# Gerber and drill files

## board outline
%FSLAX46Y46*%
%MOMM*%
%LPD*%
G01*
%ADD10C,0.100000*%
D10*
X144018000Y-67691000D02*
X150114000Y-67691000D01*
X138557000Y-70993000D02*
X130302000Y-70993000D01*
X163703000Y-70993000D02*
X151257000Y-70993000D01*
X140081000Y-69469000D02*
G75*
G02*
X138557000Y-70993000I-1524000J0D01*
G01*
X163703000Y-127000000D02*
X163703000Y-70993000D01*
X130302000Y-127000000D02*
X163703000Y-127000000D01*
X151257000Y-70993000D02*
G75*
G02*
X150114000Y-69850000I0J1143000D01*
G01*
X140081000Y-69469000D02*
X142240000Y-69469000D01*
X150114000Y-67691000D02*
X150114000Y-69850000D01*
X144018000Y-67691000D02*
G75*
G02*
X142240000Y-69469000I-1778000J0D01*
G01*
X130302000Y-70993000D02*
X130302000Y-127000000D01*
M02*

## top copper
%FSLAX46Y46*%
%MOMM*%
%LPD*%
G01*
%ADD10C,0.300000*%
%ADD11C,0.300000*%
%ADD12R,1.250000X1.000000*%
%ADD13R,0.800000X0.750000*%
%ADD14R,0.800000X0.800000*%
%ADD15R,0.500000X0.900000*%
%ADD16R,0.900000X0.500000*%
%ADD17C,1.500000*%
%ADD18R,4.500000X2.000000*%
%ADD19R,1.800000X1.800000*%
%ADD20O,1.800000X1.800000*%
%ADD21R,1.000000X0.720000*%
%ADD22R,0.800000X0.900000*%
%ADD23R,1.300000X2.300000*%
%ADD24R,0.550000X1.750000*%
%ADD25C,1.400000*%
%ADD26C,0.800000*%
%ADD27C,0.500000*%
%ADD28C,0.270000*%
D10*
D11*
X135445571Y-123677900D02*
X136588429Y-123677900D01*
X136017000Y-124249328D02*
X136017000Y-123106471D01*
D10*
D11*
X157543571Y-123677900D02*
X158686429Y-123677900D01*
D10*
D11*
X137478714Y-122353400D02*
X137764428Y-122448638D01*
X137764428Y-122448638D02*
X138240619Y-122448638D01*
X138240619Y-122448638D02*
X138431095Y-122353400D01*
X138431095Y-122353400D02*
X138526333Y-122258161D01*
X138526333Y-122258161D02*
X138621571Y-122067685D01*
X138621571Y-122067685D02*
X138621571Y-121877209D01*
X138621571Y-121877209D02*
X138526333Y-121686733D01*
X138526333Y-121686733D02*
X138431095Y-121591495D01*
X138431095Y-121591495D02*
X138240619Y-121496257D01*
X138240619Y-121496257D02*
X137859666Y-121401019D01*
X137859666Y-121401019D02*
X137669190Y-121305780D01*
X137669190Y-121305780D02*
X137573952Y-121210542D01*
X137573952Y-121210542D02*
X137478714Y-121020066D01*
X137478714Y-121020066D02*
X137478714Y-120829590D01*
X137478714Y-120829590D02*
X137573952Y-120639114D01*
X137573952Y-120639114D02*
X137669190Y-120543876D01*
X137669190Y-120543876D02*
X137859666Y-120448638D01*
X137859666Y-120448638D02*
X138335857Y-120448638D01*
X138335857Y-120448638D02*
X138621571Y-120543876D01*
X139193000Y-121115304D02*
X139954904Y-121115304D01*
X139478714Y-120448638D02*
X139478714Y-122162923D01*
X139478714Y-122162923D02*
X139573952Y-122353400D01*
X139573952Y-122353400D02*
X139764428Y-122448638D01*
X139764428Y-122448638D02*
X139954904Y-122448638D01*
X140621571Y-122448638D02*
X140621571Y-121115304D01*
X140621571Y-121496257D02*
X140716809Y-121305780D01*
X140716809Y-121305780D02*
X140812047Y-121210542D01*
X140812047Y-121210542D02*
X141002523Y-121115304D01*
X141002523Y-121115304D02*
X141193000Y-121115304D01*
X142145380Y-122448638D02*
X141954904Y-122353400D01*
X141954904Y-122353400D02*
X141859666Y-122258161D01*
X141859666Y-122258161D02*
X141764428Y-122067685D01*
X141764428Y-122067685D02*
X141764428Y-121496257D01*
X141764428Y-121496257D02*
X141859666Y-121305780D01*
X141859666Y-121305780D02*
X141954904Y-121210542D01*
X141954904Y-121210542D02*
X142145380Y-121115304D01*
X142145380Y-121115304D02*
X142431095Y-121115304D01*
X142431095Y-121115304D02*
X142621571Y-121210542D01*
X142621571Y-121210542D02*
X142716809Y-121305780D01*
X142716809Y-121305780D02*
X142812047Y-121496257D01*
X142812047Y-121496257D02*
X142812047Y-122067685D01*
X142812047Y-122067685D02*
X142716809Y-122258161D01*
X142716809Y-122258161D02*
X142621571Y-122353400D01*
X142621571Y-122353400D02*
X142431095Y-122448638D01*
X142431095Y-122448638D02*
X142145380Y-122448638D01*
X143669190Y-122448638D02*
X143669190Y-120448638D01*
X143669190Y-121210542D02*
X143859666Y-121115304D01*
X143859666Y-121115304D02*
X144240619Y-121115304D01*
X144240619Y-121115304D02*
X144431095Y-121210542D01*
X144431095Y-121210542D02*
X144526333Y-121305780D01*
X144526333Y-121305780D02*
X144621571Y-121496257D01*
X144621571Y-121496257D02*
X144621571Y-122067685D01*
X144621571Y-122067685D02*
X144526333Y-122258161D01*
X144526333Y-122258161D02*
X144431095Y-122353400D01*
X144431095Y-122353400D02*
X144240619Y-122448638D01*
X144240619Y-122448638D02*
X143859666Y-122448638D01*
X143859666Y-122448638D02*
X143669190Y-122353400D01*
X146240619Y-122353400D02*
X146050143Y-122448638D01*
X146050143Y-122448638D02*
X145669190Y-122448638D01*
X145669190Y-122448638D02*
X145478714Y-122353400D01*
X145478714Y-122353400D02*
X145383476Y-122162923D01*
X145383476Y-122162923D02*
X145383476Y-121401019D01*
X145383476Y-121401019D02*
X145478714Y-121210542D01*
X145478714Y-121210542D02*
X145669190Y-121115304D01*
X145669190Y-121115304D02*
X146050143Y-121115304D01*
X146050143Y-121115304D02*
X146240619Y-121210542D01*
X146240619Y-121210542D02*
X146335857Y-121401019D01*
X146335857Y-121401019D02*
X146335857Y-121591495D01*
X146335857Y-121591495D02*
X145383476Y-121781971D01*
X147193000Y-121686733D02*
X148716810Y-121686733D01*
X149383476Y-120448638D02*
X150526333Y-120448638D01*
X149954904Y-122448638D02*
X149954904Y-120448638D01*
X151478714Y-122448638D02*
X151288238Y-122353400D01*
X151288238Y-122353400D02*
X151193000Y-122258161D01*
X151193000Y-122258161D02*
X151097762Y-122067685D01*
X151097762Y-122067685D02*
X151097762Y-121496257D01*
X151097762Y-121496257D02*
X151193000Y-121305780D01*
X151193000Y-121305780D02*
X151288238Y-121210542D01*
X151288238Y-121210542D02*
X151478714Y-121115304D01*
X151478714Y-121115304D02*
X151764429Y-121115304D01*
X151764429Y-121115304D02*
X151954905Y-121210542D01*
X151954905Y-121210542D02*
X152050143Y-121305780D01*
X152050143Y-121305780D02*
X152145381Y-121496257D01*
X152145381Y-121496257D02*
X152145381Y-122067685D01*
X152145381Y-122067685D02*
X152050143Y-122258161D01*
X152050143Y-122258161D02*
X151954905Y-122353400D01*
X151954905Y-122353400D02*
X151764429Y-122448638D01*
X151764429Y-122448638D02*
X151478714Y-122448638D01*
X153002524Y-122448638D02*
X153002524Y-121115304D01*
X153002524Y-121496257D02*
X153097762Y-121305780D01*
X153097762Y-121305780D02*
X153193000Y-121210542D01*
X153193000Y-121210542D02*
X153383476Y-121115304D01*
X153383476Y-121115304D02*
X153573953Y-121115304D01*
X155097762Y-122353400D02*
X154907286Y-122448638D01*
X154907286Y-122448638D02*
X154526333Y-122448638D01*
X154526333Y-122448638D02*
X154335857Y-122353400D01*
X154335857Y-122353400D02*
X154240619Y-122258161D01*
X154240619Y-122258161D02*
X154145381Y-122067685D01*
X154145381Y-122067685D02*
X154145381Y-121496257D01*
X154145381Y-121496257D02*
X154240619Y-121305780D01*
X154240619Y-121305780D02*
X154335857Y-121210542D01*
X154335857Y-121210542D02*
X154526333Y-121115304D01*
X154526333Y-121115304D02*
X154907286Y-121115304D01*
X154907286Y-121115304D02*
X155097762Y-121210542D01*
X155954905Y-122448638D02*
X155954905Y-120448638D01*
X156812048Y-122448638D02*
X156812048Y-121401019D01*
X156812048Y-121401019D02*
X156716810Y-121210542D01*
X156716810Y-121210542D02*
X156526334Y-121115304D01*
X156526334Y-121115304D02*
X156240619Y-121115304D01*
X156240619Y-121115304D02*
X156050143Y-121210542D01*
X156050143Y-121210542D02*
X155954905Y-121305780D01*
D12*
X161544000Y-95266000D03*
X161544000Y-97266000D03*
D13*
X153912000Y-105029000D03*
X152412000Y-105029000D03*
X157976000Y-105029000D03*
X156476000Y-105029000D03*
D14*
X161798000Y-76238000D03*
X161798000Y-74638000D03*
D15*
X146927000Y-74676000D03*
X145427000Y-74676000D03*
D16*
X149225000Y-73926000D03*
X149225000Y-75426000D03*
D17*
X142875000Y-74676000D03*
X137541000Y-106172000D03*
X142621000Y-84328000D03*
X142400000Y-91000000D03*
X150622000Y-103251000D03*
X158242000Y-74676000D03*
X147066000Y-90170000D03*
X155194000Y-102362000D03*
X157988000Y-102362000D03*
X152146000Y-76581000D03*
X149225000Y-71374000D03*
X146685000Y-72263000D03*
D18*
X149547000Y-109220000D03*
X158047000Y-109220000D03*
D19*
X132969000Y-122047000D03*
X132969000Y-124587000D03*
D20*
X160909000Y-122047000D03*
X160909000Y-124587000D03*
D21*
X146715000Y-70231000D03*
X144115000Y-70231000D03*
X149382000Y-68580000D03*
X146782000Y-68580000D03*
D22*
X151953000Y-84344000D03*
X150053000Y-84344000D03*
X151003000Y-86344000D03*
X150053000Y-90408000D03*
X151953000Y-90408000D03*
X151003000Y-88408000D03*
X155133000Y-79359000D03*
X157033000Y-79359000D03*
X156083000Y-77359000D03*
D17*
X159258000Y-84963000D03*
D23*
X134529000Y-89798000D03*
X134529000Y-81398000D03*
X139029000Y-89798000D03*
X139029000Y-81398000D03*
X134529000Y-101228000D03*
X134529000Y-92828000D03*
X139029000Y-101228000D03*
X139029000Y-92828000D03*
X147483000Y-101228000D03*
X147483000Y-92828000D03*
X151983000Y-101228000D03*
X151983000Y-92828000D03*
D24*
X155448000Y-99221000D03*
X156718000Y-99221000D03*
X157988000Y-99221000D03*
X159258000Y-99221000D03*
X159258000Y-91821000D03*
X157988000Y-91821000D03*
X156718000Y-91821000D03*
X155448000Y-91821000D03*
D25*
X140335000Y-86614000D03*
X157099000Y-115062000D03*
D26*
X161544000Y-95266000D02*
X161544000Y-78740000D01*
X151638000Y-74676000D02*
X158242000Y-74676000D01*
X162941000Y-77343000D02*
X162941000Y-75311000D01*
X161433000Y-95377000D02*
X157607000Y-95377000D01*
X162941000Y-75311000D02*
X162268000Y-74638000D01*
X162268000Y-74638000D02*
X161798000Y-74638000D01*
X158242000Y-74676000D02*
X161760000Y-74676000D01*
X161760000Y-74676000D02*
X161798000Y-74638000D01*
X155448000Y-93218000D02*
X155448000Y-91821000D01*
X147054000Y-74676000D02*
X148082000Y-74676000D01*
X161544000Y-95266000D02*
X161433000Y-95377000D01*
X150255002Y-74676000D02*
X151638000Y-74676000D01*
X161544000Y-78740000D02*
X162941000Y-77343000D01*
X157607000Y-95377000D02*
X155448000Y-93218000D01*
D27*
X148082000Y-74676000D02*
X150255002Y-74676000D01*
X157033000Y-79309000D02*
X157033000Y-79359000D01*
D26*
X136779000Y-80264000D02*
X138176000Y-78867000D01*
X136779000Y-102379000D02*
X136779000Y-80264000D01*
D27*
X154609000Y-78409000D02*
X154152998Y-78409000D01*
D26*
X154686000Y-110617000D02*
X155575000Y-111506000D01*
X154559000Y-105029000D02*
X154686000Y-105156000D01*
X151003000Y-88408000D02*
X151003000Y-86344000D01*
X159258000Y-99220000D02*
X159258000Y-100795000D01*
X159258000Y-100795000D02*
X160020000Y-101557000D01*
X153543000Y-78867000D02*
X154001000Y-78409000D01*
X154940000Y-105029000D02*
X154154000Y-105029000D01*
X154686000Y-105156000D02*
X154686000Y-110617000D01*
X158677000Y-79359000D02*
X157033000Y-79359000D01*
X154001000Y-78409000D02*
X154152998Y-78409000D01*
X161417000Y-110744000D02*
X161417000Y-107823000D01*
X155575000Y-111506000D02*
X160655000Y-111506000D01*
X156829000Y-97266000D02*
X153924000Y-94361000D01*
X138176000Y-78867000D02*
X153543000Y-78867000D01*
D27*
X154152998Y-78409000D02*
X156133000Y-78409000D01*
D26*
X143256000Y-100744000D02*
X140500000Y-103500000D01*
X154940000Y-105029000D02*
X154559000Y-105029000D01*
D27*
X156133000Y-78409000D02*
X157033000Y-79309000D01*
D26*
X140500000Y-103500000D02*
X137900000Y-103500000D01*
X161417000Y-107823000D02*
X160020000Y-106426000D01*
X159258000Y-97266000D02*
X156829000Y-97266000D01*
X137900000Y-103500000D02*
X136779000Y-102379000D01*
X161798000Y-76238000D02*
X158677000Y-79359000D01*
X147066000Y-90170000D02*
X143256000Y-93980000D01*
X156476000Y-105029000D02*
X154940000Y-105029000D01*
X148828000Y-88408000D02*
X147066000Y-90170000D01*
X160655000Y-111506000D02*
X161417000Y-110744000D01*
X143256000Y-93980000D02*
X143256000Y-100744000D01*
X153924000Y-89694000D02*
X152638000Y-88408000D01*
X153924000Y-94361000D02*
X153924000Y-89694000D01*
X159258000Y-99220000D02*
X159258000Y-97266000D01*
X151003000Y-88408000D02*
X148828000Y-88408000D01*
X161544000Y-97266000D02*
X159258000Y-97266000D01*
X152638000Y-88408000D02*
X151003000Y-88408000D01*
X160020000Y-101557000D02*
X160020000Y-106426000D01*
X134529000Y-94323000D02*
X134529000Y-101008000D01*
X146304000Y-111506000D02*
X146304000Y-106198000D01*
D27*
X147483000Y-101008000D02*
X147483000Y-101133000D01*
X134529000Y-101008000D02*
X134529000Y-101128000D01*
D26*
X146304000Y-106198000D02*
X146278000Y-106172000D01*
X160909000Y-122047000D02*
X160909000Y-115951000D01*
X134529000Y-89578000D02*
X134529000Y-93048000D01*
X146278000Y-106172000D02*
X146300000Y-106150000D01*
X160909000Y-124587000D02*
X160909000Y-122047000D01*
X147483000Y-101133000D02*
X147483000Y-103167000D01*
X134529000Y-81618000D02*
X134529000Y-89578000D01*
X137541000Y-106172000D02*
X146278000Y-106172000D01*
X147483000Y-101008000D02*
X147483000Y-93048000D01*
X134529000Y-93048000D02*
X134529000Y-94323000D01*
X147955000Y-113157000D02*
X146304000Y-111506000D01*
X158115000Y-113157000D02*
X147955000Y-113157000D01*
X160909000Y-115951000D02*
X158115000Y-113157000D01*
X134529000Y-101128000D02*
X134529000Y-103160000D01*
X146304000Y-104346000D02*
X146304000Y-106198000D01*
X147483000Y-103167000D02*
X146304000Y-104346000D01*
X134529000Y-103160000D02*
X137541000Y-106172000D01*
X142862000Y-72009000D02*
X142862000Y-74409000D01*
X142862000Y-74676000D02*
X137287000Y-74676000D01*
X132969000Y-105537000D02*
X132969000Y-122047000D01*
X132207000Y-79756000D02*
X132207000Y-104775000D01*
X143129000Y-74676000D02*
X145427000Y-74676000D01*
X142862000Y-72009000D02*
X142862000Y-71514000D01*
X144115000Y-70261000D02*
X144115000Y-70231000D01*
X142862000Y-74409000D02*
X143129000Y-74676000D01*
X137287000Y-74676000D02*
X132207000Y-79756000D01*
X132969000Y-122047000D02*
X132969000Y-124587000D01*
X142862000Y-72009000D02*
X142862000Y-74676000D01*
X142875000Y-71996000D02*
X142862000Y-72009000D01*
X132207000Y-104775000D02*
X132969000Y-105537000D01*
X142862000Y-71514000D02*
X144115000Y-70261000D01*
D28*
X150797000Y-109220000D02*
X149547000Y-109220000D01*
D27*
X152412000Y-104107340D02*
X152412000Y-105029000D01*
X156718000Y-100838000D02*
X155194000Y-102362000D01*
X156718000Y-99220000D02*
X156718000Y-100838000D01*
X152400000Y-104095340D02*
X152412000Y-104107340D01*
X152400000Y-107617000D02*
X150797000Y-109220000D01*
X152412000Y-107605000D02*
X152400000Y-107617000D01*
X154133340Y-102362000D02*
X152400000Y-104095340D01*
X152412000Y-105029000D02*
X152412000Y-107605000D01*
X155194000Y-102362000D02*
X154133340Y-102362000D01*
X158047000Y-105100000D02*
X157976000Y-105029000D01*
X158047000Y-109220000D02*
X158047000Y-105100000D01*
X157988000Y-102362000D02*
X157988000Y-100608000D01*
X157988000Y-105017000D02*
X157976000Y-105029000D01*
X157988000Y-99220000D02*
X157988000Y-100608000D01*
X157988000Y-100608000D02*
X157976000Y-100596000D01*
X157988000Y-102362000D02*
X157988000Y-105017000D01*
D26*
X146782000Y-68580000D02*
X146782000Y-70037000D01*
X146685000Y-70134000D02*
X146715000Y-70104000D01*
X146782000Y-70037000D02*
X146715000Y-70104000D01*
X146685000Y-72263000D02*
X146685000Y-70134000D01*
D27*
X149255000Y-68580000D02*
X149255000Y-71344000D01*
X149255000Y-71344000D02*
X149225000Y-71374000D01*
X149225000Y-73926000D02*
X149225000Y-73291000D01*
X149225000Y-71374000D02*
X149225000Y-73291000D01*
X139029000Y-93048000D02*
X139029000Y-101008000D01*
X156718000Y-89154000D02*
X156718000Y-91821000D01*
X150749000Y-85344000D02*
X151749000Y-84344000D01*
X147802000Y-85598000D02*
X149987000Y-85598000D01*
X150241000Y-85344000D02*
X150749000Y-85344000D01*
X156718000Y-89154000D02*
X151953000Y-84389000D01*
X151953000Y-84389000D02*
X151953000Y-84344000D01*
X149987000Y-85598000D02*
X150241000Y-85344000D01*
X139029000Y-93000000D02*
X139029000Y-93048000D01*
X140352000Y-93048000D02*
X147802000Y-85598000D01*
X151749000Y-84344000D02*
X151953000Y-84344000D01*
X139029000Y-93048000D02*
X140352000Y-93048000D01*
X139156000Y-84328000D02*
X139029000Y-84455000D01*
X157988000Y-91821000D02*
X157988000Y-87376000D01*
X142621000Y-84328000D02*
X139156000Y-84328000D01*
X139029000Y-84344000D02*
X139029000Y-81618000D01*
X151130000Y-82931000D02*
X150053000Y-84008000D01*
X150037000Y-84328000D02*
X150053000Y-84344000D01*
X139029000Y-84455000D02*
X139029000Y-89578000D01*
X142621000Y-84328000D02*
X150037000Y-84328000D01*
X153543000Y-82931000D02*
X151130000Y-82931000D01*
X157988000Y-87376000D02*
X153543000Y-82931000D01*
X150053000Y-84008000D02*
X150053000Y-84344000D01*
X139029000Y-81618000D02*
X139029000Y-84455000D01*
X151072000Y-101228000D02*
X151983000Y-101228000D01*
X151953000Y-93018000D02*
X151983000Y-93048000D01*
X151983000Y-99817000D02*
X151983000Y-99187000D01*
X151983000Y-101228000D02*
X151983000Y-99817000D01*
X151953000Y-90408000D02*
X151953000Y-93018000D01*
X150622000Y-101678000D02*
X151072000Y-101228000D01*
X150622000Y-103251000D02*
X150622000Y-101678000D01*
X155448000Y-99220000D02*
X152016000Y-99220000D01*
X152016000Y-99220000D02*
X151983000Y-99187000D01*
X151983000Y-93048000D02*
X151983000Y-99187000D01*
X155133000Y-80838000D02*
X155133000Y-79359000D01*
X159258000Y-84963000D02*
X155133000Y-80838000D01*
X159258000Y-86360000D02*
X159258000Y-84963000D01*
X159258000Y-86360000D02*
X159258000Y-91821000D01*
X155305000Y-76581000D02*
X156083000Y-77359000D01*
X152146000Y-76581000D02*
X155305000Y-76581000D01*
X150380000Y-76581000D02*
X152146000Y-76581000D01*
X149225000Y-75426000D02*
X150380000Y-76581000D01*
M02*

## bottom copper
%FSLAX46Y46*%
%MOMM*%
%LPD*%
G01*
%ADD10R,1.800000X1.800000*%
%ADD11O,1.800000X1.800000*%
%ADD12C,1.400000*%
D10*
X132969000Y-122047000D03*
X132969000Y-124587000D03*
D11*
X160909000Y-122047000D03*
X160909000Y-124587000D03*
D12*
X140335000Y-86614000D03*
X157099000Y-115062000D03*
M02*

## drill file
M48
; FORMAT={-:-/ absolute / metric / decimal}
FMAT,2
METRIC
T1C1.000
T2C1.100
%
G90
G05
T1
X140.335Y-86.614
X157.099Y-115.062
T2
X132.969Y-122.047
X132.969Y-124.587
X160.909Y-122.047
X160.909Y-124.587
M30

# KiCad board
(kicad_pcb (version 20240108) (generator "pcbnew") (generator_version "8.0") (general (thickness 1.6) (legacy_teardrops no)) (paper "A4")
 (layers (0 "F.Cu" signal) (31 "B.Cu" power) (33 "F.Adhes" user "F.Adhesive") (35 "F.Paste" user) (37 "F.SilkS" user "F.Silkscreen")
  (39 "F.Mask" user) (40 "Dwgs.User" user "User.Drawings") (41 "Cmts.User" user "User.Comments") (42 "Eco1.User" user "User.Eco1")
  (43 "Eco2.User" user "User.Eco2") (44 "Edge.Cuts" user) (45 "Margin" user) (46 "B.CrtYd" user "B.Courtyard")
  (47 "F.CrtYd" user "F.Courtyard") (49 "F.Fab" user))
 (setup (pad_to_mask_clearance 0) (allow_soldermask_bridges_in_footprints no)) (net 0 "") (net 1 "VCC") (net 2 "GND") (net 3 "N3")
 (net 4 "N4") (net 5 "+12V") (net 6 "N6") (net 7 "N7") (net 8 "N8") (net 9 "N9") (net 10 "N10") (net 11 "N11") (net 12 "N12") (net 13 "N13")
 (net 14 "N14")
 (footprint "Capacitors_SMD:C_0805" (layer "F.Cu") (at 161.544 96.266 -90)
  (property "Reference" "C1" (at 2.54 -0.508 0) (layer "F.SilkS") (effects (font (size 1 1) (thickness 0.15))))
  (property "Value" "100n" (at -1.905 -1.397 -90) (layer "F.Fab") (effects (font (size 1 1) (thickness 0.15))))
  (pad "1" smd rect (at -1 0 270) (size 1 1.25) (layers "F.Cu" "F.Paste" "F.Mask") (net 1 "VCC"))
  (pad "2" smd rect (at 1 0 270) (size 1 1.25) (layers "F.Cu" "F.Paste" "F.Mask") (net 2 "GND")))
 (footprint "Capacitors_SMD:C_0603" (layer "F.Cu") (at 153.162 105.029 180)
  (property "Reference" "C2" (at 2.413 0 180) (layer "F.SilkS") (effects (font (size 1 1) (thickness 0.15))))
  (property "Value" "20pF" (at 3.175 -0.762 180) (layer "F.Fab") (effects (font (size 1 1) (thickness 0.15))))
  (pad "1" smd rect (at -0.75 0 180) (size 0.8 0.75) (layers "F.Cu" "F.Paste" "F.Mask") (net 2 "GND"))
  (pad "2" smd rect (at 0.75 0 180) (size 0.8 0.75) (layers "F.Cu" "F.Paste" "F.Mask") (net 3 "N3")))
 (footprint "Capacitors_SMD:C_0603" (layer "F.Cu") (at 157.226 105.029 180)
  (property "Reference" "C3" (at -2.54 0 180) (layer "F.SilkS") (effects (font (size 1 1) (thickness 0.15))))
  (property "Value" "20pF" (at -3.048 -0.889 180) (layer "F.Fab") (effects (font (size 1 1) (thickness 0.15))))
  (pad "1" smd rect (at -0.75 0 180) (size 0.8 0.75) (layers "F.Cu" "F.Paste" "F.Mask") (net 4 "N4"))
  (pad "2" smd rect (at 0.75 0 180) (size 0.8 0.75) (layers "F.Cu" "F.Paste" "F.Mask") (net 2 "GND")))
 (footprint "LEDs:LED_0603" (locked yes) (layer "F.Cu") (at 161.798 75.438 90)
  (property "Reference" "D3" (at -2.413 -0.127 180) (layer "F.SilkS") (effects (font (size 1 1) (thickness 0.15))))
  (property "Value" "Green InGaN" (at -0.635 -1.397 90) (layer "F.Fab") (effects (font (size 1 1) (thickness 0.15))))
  (pad "1" smd rect (at -0.8 0 270) (size 0.8 0.8) (layers "F.Cu" "F.Paste" "F.Mask") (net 2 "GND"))
  (pad "2" smd rect (at 0.8 0 270) (size 0.8 0.8) (layers "F.Cu" "F.Paste" "F.Mask") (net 1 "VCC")))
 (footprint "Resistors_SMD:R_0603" (layer "F.Cu") (at 146.177 74.676 180)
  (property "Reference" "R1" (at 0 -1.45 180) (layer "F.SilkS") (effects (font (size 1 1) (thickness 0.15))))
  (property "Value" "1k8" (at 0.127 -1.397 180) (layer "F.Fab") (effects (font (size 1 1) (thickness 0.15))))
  (pad "1" smd rect (at -0.75 0 180) (size 0.5 0.9) (layers "F.Cu" "F.Paste" "F.Mask") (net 1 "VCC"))
  (pad "2" smd rect (at 0.75 0 180) (size 0.5 0.9) (layers "F.Cu" "F.Paste" "F.Mask") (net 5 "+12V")))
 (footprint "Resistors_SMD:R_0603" (layer "F.Cu") (at 149.225 74.676 -90)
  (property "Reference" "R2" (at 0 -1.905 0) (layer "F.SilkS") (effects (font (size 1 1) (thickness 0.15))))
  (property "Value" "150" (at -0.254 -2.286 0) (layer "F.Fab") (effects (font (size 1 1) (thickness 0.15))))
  (pad "1" smd rect (at -0.75 0 270) (size 0.5 0.9) (layers "F.Cu" "F.Paste" "F.Mask") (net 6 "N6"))
  (pad "2" smd rect (at 0.75 0 270) (size 0.5 0.9) (layers "F.Cu" "F.Paste" "F.Mask") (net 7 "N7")))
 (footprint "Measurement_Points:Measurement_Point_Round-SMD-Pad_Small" (layer "F.Cu") (at 142.875 74.676)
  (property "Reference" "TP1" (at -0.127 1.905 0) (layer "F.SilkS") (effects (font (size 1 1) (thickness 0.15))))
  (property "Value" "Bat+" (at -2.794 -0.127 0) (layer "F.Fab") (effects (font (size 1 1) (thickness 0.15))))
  (pad "1" smd circle (at 0 0) (size 1.5 1.5) (layers "F.Cu" "F.Mask") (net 5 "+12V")))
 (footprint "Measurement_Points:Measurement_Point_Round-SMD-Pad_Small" (layer "F.Cu") (at 137.541 106.172)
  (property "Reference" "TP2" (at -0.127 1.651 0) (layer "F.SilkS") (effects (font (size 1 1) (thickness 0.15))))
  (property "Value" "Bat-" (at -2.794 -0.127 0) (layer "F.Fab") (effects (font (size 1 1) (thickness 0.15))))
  (pad "1" smd circle (at 0 0) (size 1.5 1.5) (layers "F.Cu" "F.Mask") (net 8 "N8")))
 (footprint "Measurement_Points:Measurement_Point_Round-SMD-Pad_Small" (layer "F.Cu") (at 142.621 84.328)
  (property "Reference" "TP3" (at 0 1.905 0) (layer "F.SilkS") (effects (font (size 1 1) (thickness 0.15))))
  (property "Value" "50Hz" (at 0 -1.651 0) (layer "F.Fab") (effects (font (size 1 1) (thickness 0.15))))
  (pad "1" smd circle (at 0 0) (size 1.5 1.5) (layers "F.Cu" "F.Mask") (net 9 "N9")))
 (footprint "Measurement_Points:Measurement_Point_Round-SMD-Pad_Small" (layer "F.Cu") (at 142.4 91)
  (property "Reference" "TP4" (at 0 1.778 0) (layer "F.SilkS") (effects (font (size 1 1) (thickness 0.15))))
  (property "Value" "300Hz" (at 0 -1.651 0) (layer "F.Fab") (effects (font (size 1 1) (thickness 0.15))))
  (pad "1" smd circle (at 0 0) (size 1.5 1.5) (layers "F.Cu" "F.Mask") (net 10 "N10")))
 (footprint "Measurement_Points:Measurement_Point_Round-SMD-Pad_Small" (layer "F.Cu") (at 150.622 103.251)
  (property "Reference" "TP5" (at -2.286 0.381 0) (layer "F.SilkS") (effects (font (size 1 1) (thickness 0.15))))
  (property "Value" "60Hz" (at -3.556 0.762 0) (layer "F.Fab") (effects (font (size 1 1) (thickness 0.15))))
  (pad "1" smd circle (at 0 0) (size 1.5 1.5) (layers "F.Cu" "F.Mask") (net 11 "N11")))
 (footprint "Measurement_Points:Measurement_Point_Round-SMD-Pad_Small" (layer "F.Cu") (at 158.242 74.676)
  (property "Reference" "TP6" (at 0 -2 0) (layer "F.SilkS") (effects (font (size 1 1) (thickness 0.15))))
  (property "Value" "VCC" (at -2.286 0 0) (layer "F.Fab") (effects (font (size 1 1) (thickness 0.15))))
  (pad "1" smd circle (at 0 0) (size 1.5 1.5) (layers "F.Cu" "F.Mask") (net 1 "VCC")))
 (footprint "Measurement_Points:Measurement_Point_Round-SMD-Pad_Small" (layer "F.Cu") (at 147.066 90.17)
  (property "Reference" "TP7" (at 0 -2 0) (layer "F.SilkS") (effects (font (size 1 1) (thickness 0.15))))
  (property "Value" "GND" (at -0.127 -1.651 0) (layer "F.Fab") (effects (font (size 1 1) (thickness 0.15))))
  (pad "1" smd circle (at 0 0) (size 1.5 1.5) (layers "F.Cu" "F.Mask") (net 2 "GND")))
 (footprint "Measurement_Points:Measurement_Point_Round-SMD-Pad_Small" (layer "F.Cu") (at 155.194 102.362)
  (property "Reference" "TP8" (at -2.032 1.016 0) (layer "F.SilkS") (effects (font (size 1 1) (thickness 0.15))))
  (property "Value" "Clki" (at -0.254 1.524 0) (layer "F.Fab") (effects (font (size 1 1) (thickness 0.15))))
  (pad "1" smd circle (at 0 0) (size 1.5 1.5) (layers "F.Cu" "F.Mask") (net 3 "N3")))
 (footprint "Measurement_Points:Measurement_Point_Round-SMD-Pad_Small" (layer "F.Cu") (at 157.988 102.362)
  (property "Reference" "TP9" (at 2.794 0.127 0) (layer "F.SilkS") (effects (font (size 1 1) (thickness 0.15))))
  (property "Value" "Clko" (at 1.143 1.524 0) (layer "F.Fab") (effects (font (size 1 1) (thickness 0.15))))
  (pad "1" smd circle (at 0 0) (size 1.5 1.5) (layers "F.Cu" "F.Mask") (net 4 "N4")))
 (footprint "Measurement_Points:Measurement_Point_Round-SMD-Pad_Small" (layer "F.Cu") (at 152.146 76.581)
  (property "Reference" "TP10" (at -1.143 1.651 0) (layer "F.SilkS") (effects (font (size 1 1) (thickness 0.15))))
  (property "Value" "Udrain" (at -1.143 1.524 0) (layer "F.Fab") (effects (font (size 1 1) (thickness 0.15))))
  (pad "1" smd circle (at 0 0) (size 1.5 1.5) (layers "F.Cu" "F.Mask") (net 7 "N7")))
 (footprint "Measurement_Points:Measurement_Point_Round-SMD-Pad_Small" (layer "F.Cu") (at 149.225 71.374)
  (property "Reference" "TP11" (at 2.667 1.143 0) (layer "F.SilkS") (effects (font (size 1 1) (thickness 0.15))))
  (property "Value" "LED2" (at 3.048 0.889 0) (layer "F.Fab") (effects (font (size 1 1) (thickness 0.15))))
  (pad "1" smd circle (at 0 0) (size 1.5 1.5) (layers "F.Cu" "F.Mask") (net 6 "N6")))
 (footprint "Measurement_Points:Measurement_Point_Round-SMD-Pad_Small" (layer "F.Cu") (at 146.685 72.263)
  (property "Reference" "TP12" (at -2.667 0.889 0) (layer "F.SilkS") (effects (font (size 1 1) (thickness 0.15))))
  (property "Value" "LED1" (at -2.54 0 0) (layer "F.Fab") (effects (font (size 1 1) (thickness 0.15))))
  (pad "1" smd circle (at 0 0) (size 1.5 1.5) (layers "F.Cu" "F.Mask") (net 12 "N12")))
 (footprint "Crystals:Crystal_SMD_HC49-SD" (layer "F.Cu") (at 153.797 109.22)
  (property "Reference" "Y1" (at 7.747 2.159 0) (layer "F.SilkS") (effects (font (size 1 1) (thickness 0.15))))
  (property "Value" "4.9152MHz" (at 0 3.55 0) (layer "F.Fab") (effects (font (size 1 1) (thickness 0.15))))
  (pad "1" smd rect (at -4.25 0) (size 4.5 2) (layers "F.Cu" "F.Paste" "F.Mask") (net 3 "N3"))
  (pad "2" smd rect (at 4.25 0) (size 4.5 2) (layers "F.Cu" "F.Paste" "F.Mask") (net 4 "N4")))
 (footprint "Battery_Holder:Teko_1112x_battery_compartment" (layer "F.Cu") (at 132.969 122.047)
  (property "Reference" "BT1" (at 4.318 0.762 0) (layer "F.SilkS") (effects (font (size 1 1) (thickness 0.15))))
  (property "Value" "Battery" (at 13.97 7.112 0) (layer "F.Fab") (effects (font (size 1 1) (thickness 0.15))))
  (pad "1" thru_hole rect (at 0 0) (size 1.8 1.8) (drill 1.1) (layers "*.Cu" "*.Mask") (remove_unused_layers no) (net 5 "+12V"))
  (pad "1" thru_hole rect (at 0 2.54) (size 1.8 1.8) (drill 1.1) (layers "*.Cu" "*.Mask") (remove_unused_layers no) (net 5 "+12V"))
  (pad "2" thru_hole oval (at 27.94 0) (size 1.8 1.8) (drill 1.1) (layers "*.Cu" "*.Mask") (remove_unused_layers no) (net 8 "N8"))
  (pad "2" thru_hole oval (at 27.94 2.54) (size 1.8 1.8) (drill 1.1) (layers "*.Cu" "*.Mask") (remove_unused_layers no) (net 8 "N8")))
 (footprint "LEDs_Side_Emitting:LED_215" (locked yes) (layer "F.Cu") (at 145.415 70.231)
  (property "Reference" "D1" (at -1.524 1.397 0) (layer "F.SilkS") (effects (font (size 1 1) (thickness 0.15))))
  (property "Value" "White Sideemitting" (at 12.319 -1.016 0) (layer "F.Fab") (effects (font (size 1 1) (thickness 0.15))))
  (pad "1" smd rect (at 1.3 0 180) (size 1 0.72) (layers "F.Cu" "F.Paste" "F.Mask") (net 12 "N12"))
  (pad "2" smd rect (at -1.3 0 180) (size 1 0.72) (layers "F.Cu" "F.Paste" "F.Mask") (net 5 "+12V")))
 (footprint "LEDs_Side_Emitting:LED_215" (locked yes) (layer "F.Cu") (at 148.082 68.58)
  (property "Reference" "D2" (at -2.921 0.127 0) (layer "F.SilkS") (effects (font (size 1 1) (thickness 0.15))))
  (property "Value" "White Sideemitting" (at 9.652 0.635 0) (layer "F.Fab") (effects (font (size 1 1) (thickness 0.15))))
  (pad "1" smd rect (at 1.3 0 180) (size 1 0.72) (layers "F.Cu" "F.Paste" "F.Mask") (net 6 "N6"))
  (pad "2" smd rect (at -1.3 0 180) (size 1 0.72) (layers "F.Cu" "F.Paste" "F.Mask") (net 12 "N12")))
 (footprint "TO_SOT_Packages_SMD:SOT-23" (layer "F.Cu") (at 151.003 85.344 -90)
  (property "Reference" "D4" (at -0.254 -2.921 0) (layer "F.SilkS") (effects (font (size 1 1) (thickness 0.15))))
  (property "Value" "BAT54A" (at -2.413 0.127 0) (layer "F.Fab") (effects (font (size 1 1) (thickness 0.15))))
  (pad "1" smd rect (at -1 -0.95 270) (size 0.9 0.8) (layers "F.Cu" "F.Paste" "F.Mask") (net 10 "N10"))
  (pad "2" smd rect (at -1 0.95 270) (size 0.9 0.8) (layers "F.Cu" "F.Paste" "F.Mask") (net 9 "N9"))
  (pad "3" smd rect (at 1 0 270) (size 0.9 0.8) (layers "F.Cu" "F.Paste" "F.Mask") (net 2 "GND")))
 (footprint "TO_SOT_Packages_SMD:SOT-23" (layer "F.Cu") (at 151.003 89.408 90)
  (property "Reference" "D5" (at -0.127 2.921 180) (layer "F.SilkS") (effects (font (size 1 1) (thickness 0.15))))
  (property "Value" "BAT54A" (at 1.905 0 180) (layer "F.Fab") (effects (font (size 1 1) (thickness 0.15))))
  (pad "1" smd rect (at -1 -0.95 90) (size 0.9 0.8) (layers "F.Cu" "F.Paste" "F.Mask") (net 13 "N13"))
  (pad "2" smd rect (at -1 0.95 90) (size 0.9 0.8) (layers "F.Cu" "F.Paste" "F.Mask") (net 11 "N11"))
  (pad "3" smd rect (at 1 0 90) (size 0.9 0.8) (layers "F.Cu" "F.Paste" "F.Mask") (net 2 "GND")))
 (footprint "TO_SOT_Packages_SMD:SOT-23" (layer "F.Cu") (at 156.083 78.359 90)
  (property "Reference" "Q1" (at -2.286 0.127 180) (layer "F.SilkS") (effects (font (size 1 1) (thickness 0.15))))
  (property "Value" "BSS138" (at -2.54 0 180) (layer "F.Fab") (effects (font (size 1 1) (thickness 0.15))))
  (pad "1" smd rect (at -1 -0.95 90) (size 0.9 0.8) (layers "F.Cu" "F.Paste" "F.Mask") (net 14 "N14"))
  (pad "2" smd rect (at -1 0.95 90) (size 0.9 0.8) (layers "F.Cu" "F.Paste" "F.Mask") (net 2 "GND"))
  (pad "3" smd rect (at 1 0 90) (size 0.9 0.8) (layers "F.Cu" "F.Paste" "F.Mask") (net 7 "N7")))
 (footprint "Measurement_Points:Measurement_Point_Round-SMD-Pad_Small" (layer "F.Cu") (at 159.258 84.963)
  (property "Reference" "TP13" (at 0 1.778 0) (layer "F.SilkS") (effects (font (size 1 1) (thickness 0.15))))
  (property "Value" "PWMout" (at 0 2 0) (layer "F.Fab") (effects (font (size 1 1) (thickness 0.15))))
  (pad "1" smd circle (at 0 0) (size 1.5 1.5) (layers "F.Cu" "F.Mask") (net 14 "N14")))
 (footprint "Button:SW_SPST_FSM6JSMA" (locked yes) (layer "F.Cu") (at 136.779 85.598 90)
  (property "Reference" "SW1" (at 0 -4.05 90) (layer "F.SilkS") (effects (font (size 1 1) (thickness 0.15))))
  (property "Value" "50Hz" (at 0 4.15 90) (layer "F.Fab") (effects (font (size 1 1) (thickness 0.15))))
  (pad "1" smd rect (at -4.2 -2.25 90) (size 2.3 1.3) (layers "F.Cu" "F.Paste" "F.Mask") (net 8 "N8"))
  (pad "1" smd rect (at 4.2 -2.25 90) (size 2.3 1.3) (layers "F.Cu" "F.Paste" "F.Mask") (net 8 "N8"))
  (pad "2" smd rect (at -4.2 2.25 90) (size 2.3 1.3) (layers "F.Cu" "F.Paste" "F.Mask") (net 9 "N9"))
  (pad "2" smd rect (at 4.2 2.25 90) (size 2.3 1.3) (layers "F.Cu" "F.Paste" "F.Mask") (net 9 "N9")))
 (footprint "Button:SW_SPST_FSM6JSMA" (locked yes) (layer "F.Cu") (at 136.779 97.028 90)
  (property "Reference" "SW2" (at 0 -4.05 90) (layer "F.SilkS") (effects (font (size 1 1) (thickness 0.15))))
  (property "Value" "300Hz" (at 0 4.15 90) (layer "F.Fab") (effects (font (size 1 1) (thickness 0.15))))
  (pad "1" smd rect (at -4.2 -2.25 90) (size 2.3 1.3) (layers "F.Cu" "F.Paste" "F.Mask") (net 8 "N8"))
  (pad "1" smd rect (at 4.2 -2.25 90) (size 2.3 1.3) (layers "F.Cu" "F.Paste" "F.Mask") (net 8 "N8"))
  (pad "2" smd rect (at -4.2 2.25 90) (size 2.3 1.3) (layers "F.Cu" "F.Paste" "F.Mask") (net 10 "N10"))
  (pad "2" smd rect (at 4.2 2.25 90) (size 2.3 1.3) (layers "F.Cu" "F.Paste" "F.Mask") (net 10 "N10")))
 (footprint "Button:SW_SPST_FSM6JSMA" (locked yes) (layer "F.Cu") (at 149.733 97.028 90)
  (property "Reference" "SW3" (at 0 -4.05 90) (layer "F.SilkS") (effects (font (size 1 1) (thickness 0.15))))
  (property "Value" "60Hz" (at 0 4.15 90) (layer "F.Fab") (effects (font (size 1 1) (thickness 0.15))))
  (pad "1" smd rect (at -4.2 -2.25 90) (size 2.3 1.3) (layers "F.Cu" "F.Paste" "F.Mask") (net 8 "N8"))
  (pad "1" smd rect (at 4.2 -2.25 90) (size 2.3 1.3) (layers "F.Cu" "F.Paste" "F.Mask") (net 8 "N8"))
  (pad "2" smd rect (at -4.2 2.25 90) (size 2.3 1.3) (layers "F.Cu" "F.Paste" "F.Mask") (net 11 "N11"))
  (pad "2" smd rect (at 4.2 2.25 90) (size 2.3 1.3) (layers "F.Cu" "F.Paste" "F.Mask") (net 11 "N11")))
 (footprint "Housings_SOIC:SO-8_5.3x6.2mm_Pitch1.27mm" (layer "F.Cu") (at 157.353 95.521 90)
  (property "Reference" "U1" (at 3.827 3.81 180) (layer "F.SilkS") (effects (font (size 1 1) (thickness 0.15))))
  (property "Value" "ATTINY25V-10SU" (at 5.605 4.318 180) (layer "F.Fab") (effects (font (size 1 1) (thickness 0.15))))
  (pad "1" smd rect (at -3.7 -1.905 90) (size 1.75 0.55) (layers "F.Cu" "F.Paste" "F.Mask") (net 11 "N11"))
  (pad "2" smd rect (at -3.7 -0.635 90) (size 1.75 0.55) (layers "F.Cu" "F.Paste" "F.Mask") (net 3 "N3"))
  (pad "3" smd rect (at -3.7 0.635 90) (size 1.75 0.55) (layers "F.Cu" "F.Paste" "F.Mask") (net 4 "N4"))
  (pad "4" smd rect (at -3.7 1.905 90) (size 1.75 0.55) (layers "F.Cu" "F.Paste" "F.Mask") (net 2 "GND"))
  (pad "5" smd rect (at 3.7 1.905 90) (size 1.75 0.55) (layers "F.Cu" "F.Paste" "F.Mask") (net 14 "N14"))
  (pad "6" smd rect (at 3.7 0.635 90) (size 1.75 0.55) (layers "F.Cu" "F.Paste" "F.Mask") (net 9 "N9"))
  (pad "7" smd rect (at 3.7 -0.635 90) (size 1.75 0.55) (layers "F.Cu" "F.Paste" "F.Mask") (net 10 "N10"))
  (pad "8" smd rect (at 3.7 -1.905 90) (size 1.75 0.55) (layers "F.Cu" "F.Paste" "F.Mask") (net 1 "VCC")))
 (gr_line (start 144.018 67.691) (end 150.114 67.691) (stroke (width 0.1) (type solid)) (layer "Edge.Cuts"))
 (gr_line (start 138.557 70.993) (end 130.302 70.993) (stroke (width 0.1) (type solid)) (layer "Edge.Cuts"))
 (gr_line (start 163.703 70.993) (end 151.257 70.993) (stroke (width 0.1) (type solid)) (layer "Edge.Cuts"))
 (gr_arc (start 140.081 69.469) (mid 139.634631 70.546631) (end 138.557 70.993) (stroke (width 0.1) (type solid)) (layer "Edge.Cuts"))
 (gr_line (start 163.703 127) (end 163.703 70.993) (stroke (width 0.1) (type solid)) (layer "Edge.Cuts"))
 (gr_line (start 130.302 127) (end 163.703 127) (stroke (width 0.1) (type solid)) (layer "Edge.Cuts"))
 (gr_arc (start 151.257 70.993) (mid 150.448777 70.658223) (end 150.114 69.85) (stroke (width 0.1) (type solid)) (layer "Edge.Cuts"))
 (gr_line (start 140.081 69.469) (end 142.24 69.469) (stroke (width 0.1) (type solid)) (layer "Edge.Cuts"))
 (gr_line (start 150.114 67.691) (end 150.114 69.85) (stroke (width 0.1) (type solid)) (layer "Edge.Cuts"))
 (gr_arc (start 144.018 67.691) (mid 143.497236 68.948236) (end 142.24 69.469) (stroke (width 0.1) (type solid)) (layer "Edge.Cuts"))
 (gr_line (start 130.302 70.993) (end 130.302 127) (stroke (width 0.1) (type solid)) (layer "Edge.Cuts"))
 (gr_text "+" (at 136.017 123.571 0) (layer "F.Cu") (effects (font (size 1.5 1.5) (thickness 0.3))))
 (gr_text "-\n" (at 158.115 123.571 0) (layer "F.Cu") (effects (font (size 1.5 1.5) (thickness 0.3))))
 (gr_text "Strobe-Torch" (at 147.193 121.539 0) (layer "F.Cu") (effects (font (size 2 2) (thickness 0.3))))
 (via (at 140.335 86.614) (size 1.4) (drill 1) (layers "F.Cu" "B.Cu") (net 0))
 (via (at 157.099 115.062) (size 1.4) (drill 1) (layers "F.Cu" "B.Cu") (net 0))
 (segment (start 161.544 95.266) (end 161.544 78.74) (width 0.8) (layer "F.Cu") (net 1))
 (segment (start 151.638 74.676) (end 158.242 74.676) (width 0.8) (layer "F.Cu") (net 1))
 (segment (start 162.941 77.343) (end 162.941 75.311) (width 0.8) (layer "F.Cu") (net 1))
 (segment (start 161.433 95.377) (end 157.607 95.377) (width 0.8) (layer "F.Cu") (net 1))
 (segment (start 162.941 75.311) (end 162.268 74.638) (width 0.8) (layer "F.Cu") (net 1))
 (segment (start 162.268 74.638) (end 161.798 74.638) (width 0.8) (layer "F.Cu") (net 1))
 (segment (start 158.242 74.676) (end 161.76 74.676) (width 0.8) (layer "F.Cu") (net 1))
 (segment (start 161.76 74.676) (end 161.798 74.638) (width 0.8) (layer "F.Cu") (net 1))
 (segment (start 155.448 93.218) (end 155.448 91.821) (width 0.8) (layer "F.Cu") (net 1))
 (segment (start 147.054 74.676) (end 148.082 74.676) (width 0.8) (layer "F.Cu") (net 1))
 (segment (start 161.544 95.266) (end 161.433 95.377) (width 0.8) (layer "F.Cu") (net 1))
 (segment (start 150.255002 74.676) (end 151.638 74.676) (width 0.8) (layer "F.Cu") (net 1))
 (segment (start 161.544 78.74) (end 162.941 77.343) (width 0.8) (layer "F.Cu") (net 1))
 (segment (start 157.607 95.377) (end 155.448 93.218) (width 0.8) (layer "F.Cu") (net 1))
 (segment (start 148.082 74.676) (end 150.255002 74.676) (width 0.5) (layer "F.Cu") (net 1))
 (segment (start 157.033 79.309) (end 157.033 79.359) (width 0.5) (layer "F.Cu") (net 2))
 (segment (start 136.779 80.264) (end 138.176 78.867) (width 0.8) (layer "F.Cu") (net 2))
 (segment (start 136.779 102.379) (end 136.779 80.264) (width 0.8) (layer "F.Cu") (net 2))
 (segment (start 154.609 78.409) (end 154.152998 78.409) (width 0.5) (layer "F.Cu") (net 2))
 (segment (start 154.686 110.617) (end 155.575 111.506) (width 0.8) (layer "F.Cu") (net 2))
 (segment (start 154.559 105.029) (end 154.686 105.156) (width 0.8) (layer "F.Cu") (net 2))
 (segment (start 151.003 88.408) (end 151.003 86.344) (width 0.8) (layer "F.Cu") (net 2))
 (segment (start 159.258 99.22) (end 159.258 100.795) (width 0.8) (layer "F.Cu") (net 2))
 (segment (start 159.258 100.795) (end 160.02 101.557) (width 0.8) (layer "F.Cu") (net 2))
 (segment (start 153.543 78.867) (end 154.001 78.409) (width 0.8) (layer "F.Cu") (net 2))
 (segment (start 154.94 105.029) (end 154.154 105.029) (width 0.8) (layer "F.Cu") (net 2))
 (segment (start 154.686 105.156) (end 154.686 110.617) (width 0.8) (layer "F.Cu") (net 2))
 (segment (start 158.677 79.359) (end 157.033 79.359) (width 0.8) (layer "F.Cu") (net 2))
 (segment (start 154.001 78.409) (end 154.152998 78.409) (width 0.8) (layer "F.Cu") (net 2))
 (segment (start 161.417 110.744) (end 161.417 107.823) (width 0.8) (layer "F.Cu") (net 2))
 (segment (start 155.575 111.506) (end 160.655 111.506) (width 0.8) (layer "F.Cu") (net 2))
 (segment (start 156.829 97.266) (end 153.924 94.361) (width 0.8) (layer "F.Cu") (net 2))
 (segment (start 138.176 78.867) (end 153.543 78.867) (width 0.8) (layer "F.Cu") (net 2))
 (segment (start 154.152998 78.409) (end 156.133 78.409) (width 0.5) (layer "F.Cu") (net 2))
 (segment (start 143.256 100.744) (end 140.5 103.5) (width 0.8) (layer "F.Cu") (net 2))
 (segment (start 154.94 105.029) (end 154.559 105.029) (width 0.8) (layer "F.Cu") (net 2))
 (segment (start 156.133 78.409) (end 157.033 79.309) (width 0.5) (layer "F.Cu") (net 2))
 (segment (start 140.5 103.5) (end 137.9 103.5) (width 0.8) (layer "F.Cu") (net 2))
 (segment (start 161.417 107.823) (end 160.02 106.426) (width 0.8) (layer "F.Cu") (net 2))
 (segment (start 159.258 97.266) (end 156.829 97.266) (width 0.8) (layer "F.Cu") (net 2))
 (segment (start 137.9 103.5) (end 136.779 102.379) (width 0.8) (layer "F.Cu") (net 2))
 (segment (start 161.798 76.238) (end 158.677 79.359) (width 0.8) (layer "F.Cu") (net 2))
 (segment (start 147.066 90.17) (end 143.256 93.98) (width 0.8) (layer "F.Cu") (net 2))
 (segment (start 156.476 105.029) (end 154.94 105.029) (width 0.8) (layer "F.Cu") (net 2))
 (segment (start 148.828 88.408) (end 147.066 90.17) (width 0.8) (layer "F.Cu") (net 2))
 (segment (start 160.655 111.506) (end 161.417 110.744) (width 0.8) (layer "F.Cu") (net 2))
 (segment (start 143.256 93.98) (end 143.256 100.744) (width 0.8) (layer "F.Cu") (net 2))
 (segment (start 153.924 89.694) (end 152.638 88.408) (width 0.8) (layer "F.Cu") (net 2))
 (segment (start 153.924 94.361) (end 153.924 89.694) (width 0.8) (layer "F.Cu") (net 2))
 (segment (start 159.258 99.22) (end 159.258 97.266) (width 0.8) (layer "F.Cu") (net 2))
 (segment (start 151.003 88.408) (end 148.828 88.408) (width 0.8) (layer "F.Cu") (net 2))
 (segment (start 161.544 97.266) (end 159.258 97.266) (width 0.8) (layer "F.Cu") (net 2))
 (segment (start 152.638 88.408) (end 151.003 88.408) (width 0.8) (layer "F.Cu") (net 2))
 (segment (start 160.02 101.557) (end 160.02 106.426) (width 0.8) (layer "F.Cu") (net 2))
 (segment (start 134.529 94.323) (end 134.529 101.008) (width 0.8) (layer "F.Cu") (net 8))
 (segment (start 146.304 111.506) (end 146.304 106.198) (width 0.8) (layer "F.Cu") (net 8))
 (segment (start 147.483 101.008) (end 147.483 101.133) (width 0.5) (layer "F.Cu") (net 8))
 (segment (start 134.529 101.008) (end 134.529 101.128) (width 0.5) (layer "F.Cu") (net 8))
 (segment (start 146.304 106.198) (end 146.278 106.172) (width 0.8) (layer "F.Cu") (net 8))
 (segment (start 160.909 122.047) (end 160.909 115.951) (width 0.8) (layer "F.Cu") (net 8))
 (segment (start 134.529 89.578) (end 134.529 93.048) (width 0.8) (layer "F.Cu") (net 8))
 (segment (start 146.278 106.172) (end 146.3 106.15) (width 0.8) (layer "F.Cu") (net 8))
 (segment (start 160.909 124.587) (end 160.909 122.047) (width 0.8) (layer "F.Cu") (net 8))
 (segment (start 147.483 101.133) (end 147.483 103.167) (width 0.8) (layer "F.Cu") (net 8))
 (segment (start 134.529 81.618) (end 134.529 89.578) (width 0.8) (layer "F.Cu") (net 8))
 (segment (start 137.541 106.172) (end 146.278 106.172) (width 0.8) (layer "F.Cu") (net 8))
 (segment (start 147.483 101.008) (end 147.483 93.048) (width 0.8) (layer "F.Cu") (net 8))
 (segment (start 134.529 93.048) (end 134.529 94.323) (width 0.8) (layer "F.Cu") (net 8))
 (segment (start 147.955 113.157) (end 146.304 111.506) (width 0.8) (layer "F.Cu") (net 8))
 (segment (start 158.115 113.157) (end 147.955 113.157) (width 0.8) (layer "F.Cu") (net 8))
 (segment (start 160.909 115.951) (end 158.115 113.157) (width 0.8) (layer "F.Cu") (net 8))
 (segment (start 134.529 101.128) (end 134.529 103.16) (width 0.8) (layer "F.Cu") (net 8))
 (segment (start 146.304 104.346) (end 146.304 106.198) (width 0.8) (layer "F.Cu") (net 8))
 (segment (start 147.483 103.167) (end 146.304 104.346) (width 0.8) (layer "F.Cu") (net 8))
 (segment (start 134.529 103.16) (end 137.541 106.172) (width 0.8) (layer "F.Cu") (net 8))
 (segment (start 142.862 72.009) (end 142.862 74.409) (width 0.8) (layer "F.Cu") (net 5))
 (segment (start 142.862 74.676) (end 137.287 74.676) (width 0.8) (layer "F.Cu") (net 5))
 (segment (start 132.969 105.537) (end 132.969 122.047) (width 0.8) (layer "F.Cu") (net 5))
 (segment (start 132.207 79.756) (end 132.207 104.775) (width 0.8) (layer "F.Cu") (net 5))
 (segment (start 143.129 74.676) (end 145.427 74.676) (width 0.8) (layer "F.Cu") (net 5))
 (segment (start 142.862 72.009) (end 142.862 71.514) (width 0.8) (layer "F.Cu") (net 5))
 (segment (start 144.115 70.261) (end 144.115 70.231) (width 0.8) (layer "F.Cu") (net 5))
 (segment (start 142.862 74.409) (end 143.129 74.676) (width 0.8) (layer "F.Cu") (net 5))
 (segment (start 137.287 74.676) (end 132.207 79.756) (width 0.8) (layer "F.Cu") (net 5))
 (segment (start 132.969 122.047) (end 132.969 124.587) (width 0.8) (layer "F.Cu") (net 5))
 (segment (start 142.862 72.009) (end 142.862 74.676) (width 0.8) (layer "F.Cu") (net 5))
 (segment (start 142.875 71.996) (end 142.862 72.009) (width 0.8) (layer "F.Cu") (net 5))
 (segment (start 132.207 104.775) (end 132.969 105.537) (width 0.8) (layer "F.Cu") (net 5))
 (segment (start 142.862 71.514) (end 144.115 70.261) (width 0.8) (layer "F.Cu") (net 5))
 (segment (start 150.797 109.22) (end 149.547 109.22) (width 0.27) (layer "F.Cu") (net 3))
 (segment (start 152.412 104.10734) (end 152.412 105.029) (width 0.5) (layer "F.Cu") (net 3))
 (segment (start 156.718 100.838) (end 155.194 102.362) (width 0.5) (layer "F.Cu") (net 3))
 (segment (start 156.718 99.22) (end 156.718 100.838) (width 0.5) (layer "F.Cu") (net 3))
 (segment (start 152.4 104.09534) (end 152.412 104.10734) (width 0.5) (layer "F.Cu") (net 3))
 (segment (start 152.4 107.617) (end 150.797 109.22) (width 0.5) (layer "F.Cu") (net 3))
 (segment (start 152.412 107.605) (end 152.4 107.617) (width 0.5) (layer "F.Cu") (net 3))
 (segment (start 154.13334 102.362) (end 152.4 104.09534) (width 0.5) (layer "F.Cu") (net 3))
 (segment (start 152.412 105.029) (end 152.412 107.605) (width 0.5) (layer "F.Cu") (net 3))
 (segment (start 155.194 102.362) (end 154.13334 102.362) (width 0.5) (layer "F.Cu") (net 3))
 (segment (start 158.047 105.1) (end 157.976 105.029) (width 0.5) (layer "F.Cu") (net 4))
 (segment (start 158.047 109.22) (end 158.047 105.1) (width 0.5) (layer "F.Cu") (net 4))
 (segment (start 157.988 102.362) (end 157.988 100.608) (width 0.5) (layer "F.Cu") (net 4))
 (segment (start 157.988 105.017) (end 157.976 105.029) (width 0.5) (layer "F.Cu") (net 4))
 (segment (start 157.988 99.22) (end 157.988 100.608) (width 0.5) (layer "F.Cu") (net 4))
 (segment (start 157.988 100.608) (end 157.976 100.596) (width 0.5) (layer "F.Cu") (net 4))
 (segment (start 157.988 102.362) (end 157.988 105.017) (width 0.5) (layer "F.Cu") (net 4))
 (segment (start 146.782 68.58) (end 146.782 70.037) (width 0.8) (layer "F.Cu") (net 12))
 (segment (start 146.685 70.134) (end 146.715 70.104) (width 0.8) (layer "F.Cu") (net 12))
 (segment (start 146.782 70.037) (end 146.715 70.104) (width 0.8) (layer "F.Cu") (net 12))
 (segment (start 146.685 72.263) (end 146.685 70.134) (width 0.8) (layer "F.Cu") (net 12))
 (segment (start 149.255 68.58) (end 149.255 71.344) (width 0.5) (layer "F.Cu") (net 6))
 (segment (start 149.255 71.344) (end 149.225 71.374) (width 0.5) (layer "F.Cu") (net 6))
 (segment (start 149.225 73.926) (end 149.225 73.291) (width 0.5) (layer "F.Cu") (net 6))
 (segment (start 149.225 71.374) (end 149.225 73.291) (width 0.5) (layer "F.Cu") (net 6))
 (segment (start 139.029 93.048) (end 139.029 101.008) (width 0.5) (layer "F.Cu") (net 10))
 (segment (start 156.718 89.154) (end 156.718 91.821) (width 0.5) (layer "F.Cu") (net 10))
 (segment (start 150.749 85.344) (end 151.749 84.344) (width 0.5) (layer "F.Cu") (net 10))
 (segment (start 147.802 85.598) (end 149.987 85.598) (width 0.5) (layer "F.Cu") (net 10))
 (segment (start 150.241 85.344) (end 150.749 85.344) (width 0.5) (layer "F.Cu") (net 10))
 (segment (start 156.718 89.154) (end 151.953 84.389) (width 0.5) (layer "F.Cu") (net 10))
 (segment (start 151.953 84.389) (end 151.953 84.344) (width 0.5) (layer "F.Cu") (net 10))
 (segment (start 149.987 85.598) (end 150.241 85.344) (width 0.5) (layer "F.Cu") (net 10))
 (segment (start 139.029 93) (end 139.029 93.048) (width 0.5) (layer "F.Cu") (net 10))
 (segment (start 140.352 93.048) (end 147.802 85.598) (width 0.5) (layer "F.Cu") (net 10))
 (segment (start 151.749 84.344) (end 151.953 84.344) (width 0.5) (layer "F.Cu") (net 10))
 (segment (start 139.029 93.048) (end 140.352 93.048) (width 0.5) (layer "F.Cu") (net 10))
 (segment (start 139.156 84.328) (end 139.029 84.455) (width 0.5) (layer "F.Cu") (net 9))
 (segment (start 157.988 91.821) (end 157.988 87.376) (width 0.5) (layer "F.Cu") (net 9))
 (segment (start 142.621 84.328) (end 139.156 84.328) (width 0.5) (layer "F.Cu") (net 9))
 (segment (start 139.029 84.344) (end 139.029 81.618) (width 0.5) (layer "F.Cu") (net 9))
 (segment (start 151.13 82.931) (end 150.053 84.008) (width 0.5) (layer "F.Cu") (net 9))
 (segment (start 150.037 84.328) (end 150.053 84.344) (width 0.5) (layer "F.Cu") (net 9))
 (segment (start 139.029 84.455) (end 139.029 89.578) (width 0.5) (layer "F.Cu") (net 9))
 (segment (start 142.621 84.328) (end 150.037 84.328) (width 0.5) (layer "F.Cu") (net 9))
 (segment (start 153.543 82.931) (end 151.13 82.931) (width 0.5) (layer "F.Cu") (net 9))
 (segment (start 157.988 87.376) (end 153.543 82.931) (width 0.5) (layer "F.Cu") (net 9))
 (segment (start 150.053 84.008) (end 150.053 84.344) (width 0.5) (layer "F.Cu") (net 9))
 (segment (start 139.029 81.618) (end 139.029 84.455) (width 0.5) (layer "F.Cu") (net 9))
 (segment (start 151.072 101.228) (end 151.983 101.228) (width 0.5) (layer "F.Cu") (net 11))
 (segment (start 151.953 93.018) (end 151.983 93.048) (width 0.5) (layer "F.Cu") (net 11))
 (segment (start 151.983 99.817) (end 151.983 99.187) (width 0.5) (layer "F.Cu") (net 11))
 (segment (start 151.983 101.228) (end 151.983 99.817) (width 0.5) (layer "F.Cu") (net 11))
 (segment (start 151.953 90.408) (end 151.953 93.018) (width 0.5) (layer "F.Cu") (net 11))
 (segment (start 150.622 101.678) (end 151.072 101.228) (width 0.5) (layer "F.Cu") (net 11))
 (segment (start 150.622 103.251) (end 150.622 101.678) (width 0.5) (layer "F.Cu") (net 11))
 (segment (start 155.448 99.22) (end 152.016 99.22) (width 0.5) (layer "F.Cu") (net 11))
 (segment (start 152.016 99.22) (end 151.983 99.187) (width 0.5) (layer "F.Cu") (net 11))
 (segment (start 151.983 93.048) (end 151.983 99.187) (width 0.5) (layer "F.Cu") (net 11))
 (segment (start 155.133 80.838) (end 155.133 79.359) (width 0.5) (layer "F.Cu") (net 14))
 (segment (start 159.258 84.963) (end 155.133 80.838) (width 0.5) (layer "F.Cu") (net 14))
 (segment (start 159.258 86.36) (end 159.258 84.963) (width 0.5) (layer "F.Cu") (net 14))
 (segment (start 159.258 86.36) (end 159.258 91.821) (width 0.5) (layer "F.Cu") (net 14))
 (segment (start 155.305 76.581) (end 156.083 77.359) (width 0.5) (layer "F.Cu") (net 7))
 (segment (start 152.146 76.581) (end 155.305 76.581) (width 0.5) (layer "F.Cu") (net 7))
 (segment (start 150.38 76.581) (end 152.146 76.581) (width 0.5) (layer "F.Cu") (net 7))
 (segment (start 149.225 75.426) (end 150.38 76.581) (width 0.5) (layer "F.Cu") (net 7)))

